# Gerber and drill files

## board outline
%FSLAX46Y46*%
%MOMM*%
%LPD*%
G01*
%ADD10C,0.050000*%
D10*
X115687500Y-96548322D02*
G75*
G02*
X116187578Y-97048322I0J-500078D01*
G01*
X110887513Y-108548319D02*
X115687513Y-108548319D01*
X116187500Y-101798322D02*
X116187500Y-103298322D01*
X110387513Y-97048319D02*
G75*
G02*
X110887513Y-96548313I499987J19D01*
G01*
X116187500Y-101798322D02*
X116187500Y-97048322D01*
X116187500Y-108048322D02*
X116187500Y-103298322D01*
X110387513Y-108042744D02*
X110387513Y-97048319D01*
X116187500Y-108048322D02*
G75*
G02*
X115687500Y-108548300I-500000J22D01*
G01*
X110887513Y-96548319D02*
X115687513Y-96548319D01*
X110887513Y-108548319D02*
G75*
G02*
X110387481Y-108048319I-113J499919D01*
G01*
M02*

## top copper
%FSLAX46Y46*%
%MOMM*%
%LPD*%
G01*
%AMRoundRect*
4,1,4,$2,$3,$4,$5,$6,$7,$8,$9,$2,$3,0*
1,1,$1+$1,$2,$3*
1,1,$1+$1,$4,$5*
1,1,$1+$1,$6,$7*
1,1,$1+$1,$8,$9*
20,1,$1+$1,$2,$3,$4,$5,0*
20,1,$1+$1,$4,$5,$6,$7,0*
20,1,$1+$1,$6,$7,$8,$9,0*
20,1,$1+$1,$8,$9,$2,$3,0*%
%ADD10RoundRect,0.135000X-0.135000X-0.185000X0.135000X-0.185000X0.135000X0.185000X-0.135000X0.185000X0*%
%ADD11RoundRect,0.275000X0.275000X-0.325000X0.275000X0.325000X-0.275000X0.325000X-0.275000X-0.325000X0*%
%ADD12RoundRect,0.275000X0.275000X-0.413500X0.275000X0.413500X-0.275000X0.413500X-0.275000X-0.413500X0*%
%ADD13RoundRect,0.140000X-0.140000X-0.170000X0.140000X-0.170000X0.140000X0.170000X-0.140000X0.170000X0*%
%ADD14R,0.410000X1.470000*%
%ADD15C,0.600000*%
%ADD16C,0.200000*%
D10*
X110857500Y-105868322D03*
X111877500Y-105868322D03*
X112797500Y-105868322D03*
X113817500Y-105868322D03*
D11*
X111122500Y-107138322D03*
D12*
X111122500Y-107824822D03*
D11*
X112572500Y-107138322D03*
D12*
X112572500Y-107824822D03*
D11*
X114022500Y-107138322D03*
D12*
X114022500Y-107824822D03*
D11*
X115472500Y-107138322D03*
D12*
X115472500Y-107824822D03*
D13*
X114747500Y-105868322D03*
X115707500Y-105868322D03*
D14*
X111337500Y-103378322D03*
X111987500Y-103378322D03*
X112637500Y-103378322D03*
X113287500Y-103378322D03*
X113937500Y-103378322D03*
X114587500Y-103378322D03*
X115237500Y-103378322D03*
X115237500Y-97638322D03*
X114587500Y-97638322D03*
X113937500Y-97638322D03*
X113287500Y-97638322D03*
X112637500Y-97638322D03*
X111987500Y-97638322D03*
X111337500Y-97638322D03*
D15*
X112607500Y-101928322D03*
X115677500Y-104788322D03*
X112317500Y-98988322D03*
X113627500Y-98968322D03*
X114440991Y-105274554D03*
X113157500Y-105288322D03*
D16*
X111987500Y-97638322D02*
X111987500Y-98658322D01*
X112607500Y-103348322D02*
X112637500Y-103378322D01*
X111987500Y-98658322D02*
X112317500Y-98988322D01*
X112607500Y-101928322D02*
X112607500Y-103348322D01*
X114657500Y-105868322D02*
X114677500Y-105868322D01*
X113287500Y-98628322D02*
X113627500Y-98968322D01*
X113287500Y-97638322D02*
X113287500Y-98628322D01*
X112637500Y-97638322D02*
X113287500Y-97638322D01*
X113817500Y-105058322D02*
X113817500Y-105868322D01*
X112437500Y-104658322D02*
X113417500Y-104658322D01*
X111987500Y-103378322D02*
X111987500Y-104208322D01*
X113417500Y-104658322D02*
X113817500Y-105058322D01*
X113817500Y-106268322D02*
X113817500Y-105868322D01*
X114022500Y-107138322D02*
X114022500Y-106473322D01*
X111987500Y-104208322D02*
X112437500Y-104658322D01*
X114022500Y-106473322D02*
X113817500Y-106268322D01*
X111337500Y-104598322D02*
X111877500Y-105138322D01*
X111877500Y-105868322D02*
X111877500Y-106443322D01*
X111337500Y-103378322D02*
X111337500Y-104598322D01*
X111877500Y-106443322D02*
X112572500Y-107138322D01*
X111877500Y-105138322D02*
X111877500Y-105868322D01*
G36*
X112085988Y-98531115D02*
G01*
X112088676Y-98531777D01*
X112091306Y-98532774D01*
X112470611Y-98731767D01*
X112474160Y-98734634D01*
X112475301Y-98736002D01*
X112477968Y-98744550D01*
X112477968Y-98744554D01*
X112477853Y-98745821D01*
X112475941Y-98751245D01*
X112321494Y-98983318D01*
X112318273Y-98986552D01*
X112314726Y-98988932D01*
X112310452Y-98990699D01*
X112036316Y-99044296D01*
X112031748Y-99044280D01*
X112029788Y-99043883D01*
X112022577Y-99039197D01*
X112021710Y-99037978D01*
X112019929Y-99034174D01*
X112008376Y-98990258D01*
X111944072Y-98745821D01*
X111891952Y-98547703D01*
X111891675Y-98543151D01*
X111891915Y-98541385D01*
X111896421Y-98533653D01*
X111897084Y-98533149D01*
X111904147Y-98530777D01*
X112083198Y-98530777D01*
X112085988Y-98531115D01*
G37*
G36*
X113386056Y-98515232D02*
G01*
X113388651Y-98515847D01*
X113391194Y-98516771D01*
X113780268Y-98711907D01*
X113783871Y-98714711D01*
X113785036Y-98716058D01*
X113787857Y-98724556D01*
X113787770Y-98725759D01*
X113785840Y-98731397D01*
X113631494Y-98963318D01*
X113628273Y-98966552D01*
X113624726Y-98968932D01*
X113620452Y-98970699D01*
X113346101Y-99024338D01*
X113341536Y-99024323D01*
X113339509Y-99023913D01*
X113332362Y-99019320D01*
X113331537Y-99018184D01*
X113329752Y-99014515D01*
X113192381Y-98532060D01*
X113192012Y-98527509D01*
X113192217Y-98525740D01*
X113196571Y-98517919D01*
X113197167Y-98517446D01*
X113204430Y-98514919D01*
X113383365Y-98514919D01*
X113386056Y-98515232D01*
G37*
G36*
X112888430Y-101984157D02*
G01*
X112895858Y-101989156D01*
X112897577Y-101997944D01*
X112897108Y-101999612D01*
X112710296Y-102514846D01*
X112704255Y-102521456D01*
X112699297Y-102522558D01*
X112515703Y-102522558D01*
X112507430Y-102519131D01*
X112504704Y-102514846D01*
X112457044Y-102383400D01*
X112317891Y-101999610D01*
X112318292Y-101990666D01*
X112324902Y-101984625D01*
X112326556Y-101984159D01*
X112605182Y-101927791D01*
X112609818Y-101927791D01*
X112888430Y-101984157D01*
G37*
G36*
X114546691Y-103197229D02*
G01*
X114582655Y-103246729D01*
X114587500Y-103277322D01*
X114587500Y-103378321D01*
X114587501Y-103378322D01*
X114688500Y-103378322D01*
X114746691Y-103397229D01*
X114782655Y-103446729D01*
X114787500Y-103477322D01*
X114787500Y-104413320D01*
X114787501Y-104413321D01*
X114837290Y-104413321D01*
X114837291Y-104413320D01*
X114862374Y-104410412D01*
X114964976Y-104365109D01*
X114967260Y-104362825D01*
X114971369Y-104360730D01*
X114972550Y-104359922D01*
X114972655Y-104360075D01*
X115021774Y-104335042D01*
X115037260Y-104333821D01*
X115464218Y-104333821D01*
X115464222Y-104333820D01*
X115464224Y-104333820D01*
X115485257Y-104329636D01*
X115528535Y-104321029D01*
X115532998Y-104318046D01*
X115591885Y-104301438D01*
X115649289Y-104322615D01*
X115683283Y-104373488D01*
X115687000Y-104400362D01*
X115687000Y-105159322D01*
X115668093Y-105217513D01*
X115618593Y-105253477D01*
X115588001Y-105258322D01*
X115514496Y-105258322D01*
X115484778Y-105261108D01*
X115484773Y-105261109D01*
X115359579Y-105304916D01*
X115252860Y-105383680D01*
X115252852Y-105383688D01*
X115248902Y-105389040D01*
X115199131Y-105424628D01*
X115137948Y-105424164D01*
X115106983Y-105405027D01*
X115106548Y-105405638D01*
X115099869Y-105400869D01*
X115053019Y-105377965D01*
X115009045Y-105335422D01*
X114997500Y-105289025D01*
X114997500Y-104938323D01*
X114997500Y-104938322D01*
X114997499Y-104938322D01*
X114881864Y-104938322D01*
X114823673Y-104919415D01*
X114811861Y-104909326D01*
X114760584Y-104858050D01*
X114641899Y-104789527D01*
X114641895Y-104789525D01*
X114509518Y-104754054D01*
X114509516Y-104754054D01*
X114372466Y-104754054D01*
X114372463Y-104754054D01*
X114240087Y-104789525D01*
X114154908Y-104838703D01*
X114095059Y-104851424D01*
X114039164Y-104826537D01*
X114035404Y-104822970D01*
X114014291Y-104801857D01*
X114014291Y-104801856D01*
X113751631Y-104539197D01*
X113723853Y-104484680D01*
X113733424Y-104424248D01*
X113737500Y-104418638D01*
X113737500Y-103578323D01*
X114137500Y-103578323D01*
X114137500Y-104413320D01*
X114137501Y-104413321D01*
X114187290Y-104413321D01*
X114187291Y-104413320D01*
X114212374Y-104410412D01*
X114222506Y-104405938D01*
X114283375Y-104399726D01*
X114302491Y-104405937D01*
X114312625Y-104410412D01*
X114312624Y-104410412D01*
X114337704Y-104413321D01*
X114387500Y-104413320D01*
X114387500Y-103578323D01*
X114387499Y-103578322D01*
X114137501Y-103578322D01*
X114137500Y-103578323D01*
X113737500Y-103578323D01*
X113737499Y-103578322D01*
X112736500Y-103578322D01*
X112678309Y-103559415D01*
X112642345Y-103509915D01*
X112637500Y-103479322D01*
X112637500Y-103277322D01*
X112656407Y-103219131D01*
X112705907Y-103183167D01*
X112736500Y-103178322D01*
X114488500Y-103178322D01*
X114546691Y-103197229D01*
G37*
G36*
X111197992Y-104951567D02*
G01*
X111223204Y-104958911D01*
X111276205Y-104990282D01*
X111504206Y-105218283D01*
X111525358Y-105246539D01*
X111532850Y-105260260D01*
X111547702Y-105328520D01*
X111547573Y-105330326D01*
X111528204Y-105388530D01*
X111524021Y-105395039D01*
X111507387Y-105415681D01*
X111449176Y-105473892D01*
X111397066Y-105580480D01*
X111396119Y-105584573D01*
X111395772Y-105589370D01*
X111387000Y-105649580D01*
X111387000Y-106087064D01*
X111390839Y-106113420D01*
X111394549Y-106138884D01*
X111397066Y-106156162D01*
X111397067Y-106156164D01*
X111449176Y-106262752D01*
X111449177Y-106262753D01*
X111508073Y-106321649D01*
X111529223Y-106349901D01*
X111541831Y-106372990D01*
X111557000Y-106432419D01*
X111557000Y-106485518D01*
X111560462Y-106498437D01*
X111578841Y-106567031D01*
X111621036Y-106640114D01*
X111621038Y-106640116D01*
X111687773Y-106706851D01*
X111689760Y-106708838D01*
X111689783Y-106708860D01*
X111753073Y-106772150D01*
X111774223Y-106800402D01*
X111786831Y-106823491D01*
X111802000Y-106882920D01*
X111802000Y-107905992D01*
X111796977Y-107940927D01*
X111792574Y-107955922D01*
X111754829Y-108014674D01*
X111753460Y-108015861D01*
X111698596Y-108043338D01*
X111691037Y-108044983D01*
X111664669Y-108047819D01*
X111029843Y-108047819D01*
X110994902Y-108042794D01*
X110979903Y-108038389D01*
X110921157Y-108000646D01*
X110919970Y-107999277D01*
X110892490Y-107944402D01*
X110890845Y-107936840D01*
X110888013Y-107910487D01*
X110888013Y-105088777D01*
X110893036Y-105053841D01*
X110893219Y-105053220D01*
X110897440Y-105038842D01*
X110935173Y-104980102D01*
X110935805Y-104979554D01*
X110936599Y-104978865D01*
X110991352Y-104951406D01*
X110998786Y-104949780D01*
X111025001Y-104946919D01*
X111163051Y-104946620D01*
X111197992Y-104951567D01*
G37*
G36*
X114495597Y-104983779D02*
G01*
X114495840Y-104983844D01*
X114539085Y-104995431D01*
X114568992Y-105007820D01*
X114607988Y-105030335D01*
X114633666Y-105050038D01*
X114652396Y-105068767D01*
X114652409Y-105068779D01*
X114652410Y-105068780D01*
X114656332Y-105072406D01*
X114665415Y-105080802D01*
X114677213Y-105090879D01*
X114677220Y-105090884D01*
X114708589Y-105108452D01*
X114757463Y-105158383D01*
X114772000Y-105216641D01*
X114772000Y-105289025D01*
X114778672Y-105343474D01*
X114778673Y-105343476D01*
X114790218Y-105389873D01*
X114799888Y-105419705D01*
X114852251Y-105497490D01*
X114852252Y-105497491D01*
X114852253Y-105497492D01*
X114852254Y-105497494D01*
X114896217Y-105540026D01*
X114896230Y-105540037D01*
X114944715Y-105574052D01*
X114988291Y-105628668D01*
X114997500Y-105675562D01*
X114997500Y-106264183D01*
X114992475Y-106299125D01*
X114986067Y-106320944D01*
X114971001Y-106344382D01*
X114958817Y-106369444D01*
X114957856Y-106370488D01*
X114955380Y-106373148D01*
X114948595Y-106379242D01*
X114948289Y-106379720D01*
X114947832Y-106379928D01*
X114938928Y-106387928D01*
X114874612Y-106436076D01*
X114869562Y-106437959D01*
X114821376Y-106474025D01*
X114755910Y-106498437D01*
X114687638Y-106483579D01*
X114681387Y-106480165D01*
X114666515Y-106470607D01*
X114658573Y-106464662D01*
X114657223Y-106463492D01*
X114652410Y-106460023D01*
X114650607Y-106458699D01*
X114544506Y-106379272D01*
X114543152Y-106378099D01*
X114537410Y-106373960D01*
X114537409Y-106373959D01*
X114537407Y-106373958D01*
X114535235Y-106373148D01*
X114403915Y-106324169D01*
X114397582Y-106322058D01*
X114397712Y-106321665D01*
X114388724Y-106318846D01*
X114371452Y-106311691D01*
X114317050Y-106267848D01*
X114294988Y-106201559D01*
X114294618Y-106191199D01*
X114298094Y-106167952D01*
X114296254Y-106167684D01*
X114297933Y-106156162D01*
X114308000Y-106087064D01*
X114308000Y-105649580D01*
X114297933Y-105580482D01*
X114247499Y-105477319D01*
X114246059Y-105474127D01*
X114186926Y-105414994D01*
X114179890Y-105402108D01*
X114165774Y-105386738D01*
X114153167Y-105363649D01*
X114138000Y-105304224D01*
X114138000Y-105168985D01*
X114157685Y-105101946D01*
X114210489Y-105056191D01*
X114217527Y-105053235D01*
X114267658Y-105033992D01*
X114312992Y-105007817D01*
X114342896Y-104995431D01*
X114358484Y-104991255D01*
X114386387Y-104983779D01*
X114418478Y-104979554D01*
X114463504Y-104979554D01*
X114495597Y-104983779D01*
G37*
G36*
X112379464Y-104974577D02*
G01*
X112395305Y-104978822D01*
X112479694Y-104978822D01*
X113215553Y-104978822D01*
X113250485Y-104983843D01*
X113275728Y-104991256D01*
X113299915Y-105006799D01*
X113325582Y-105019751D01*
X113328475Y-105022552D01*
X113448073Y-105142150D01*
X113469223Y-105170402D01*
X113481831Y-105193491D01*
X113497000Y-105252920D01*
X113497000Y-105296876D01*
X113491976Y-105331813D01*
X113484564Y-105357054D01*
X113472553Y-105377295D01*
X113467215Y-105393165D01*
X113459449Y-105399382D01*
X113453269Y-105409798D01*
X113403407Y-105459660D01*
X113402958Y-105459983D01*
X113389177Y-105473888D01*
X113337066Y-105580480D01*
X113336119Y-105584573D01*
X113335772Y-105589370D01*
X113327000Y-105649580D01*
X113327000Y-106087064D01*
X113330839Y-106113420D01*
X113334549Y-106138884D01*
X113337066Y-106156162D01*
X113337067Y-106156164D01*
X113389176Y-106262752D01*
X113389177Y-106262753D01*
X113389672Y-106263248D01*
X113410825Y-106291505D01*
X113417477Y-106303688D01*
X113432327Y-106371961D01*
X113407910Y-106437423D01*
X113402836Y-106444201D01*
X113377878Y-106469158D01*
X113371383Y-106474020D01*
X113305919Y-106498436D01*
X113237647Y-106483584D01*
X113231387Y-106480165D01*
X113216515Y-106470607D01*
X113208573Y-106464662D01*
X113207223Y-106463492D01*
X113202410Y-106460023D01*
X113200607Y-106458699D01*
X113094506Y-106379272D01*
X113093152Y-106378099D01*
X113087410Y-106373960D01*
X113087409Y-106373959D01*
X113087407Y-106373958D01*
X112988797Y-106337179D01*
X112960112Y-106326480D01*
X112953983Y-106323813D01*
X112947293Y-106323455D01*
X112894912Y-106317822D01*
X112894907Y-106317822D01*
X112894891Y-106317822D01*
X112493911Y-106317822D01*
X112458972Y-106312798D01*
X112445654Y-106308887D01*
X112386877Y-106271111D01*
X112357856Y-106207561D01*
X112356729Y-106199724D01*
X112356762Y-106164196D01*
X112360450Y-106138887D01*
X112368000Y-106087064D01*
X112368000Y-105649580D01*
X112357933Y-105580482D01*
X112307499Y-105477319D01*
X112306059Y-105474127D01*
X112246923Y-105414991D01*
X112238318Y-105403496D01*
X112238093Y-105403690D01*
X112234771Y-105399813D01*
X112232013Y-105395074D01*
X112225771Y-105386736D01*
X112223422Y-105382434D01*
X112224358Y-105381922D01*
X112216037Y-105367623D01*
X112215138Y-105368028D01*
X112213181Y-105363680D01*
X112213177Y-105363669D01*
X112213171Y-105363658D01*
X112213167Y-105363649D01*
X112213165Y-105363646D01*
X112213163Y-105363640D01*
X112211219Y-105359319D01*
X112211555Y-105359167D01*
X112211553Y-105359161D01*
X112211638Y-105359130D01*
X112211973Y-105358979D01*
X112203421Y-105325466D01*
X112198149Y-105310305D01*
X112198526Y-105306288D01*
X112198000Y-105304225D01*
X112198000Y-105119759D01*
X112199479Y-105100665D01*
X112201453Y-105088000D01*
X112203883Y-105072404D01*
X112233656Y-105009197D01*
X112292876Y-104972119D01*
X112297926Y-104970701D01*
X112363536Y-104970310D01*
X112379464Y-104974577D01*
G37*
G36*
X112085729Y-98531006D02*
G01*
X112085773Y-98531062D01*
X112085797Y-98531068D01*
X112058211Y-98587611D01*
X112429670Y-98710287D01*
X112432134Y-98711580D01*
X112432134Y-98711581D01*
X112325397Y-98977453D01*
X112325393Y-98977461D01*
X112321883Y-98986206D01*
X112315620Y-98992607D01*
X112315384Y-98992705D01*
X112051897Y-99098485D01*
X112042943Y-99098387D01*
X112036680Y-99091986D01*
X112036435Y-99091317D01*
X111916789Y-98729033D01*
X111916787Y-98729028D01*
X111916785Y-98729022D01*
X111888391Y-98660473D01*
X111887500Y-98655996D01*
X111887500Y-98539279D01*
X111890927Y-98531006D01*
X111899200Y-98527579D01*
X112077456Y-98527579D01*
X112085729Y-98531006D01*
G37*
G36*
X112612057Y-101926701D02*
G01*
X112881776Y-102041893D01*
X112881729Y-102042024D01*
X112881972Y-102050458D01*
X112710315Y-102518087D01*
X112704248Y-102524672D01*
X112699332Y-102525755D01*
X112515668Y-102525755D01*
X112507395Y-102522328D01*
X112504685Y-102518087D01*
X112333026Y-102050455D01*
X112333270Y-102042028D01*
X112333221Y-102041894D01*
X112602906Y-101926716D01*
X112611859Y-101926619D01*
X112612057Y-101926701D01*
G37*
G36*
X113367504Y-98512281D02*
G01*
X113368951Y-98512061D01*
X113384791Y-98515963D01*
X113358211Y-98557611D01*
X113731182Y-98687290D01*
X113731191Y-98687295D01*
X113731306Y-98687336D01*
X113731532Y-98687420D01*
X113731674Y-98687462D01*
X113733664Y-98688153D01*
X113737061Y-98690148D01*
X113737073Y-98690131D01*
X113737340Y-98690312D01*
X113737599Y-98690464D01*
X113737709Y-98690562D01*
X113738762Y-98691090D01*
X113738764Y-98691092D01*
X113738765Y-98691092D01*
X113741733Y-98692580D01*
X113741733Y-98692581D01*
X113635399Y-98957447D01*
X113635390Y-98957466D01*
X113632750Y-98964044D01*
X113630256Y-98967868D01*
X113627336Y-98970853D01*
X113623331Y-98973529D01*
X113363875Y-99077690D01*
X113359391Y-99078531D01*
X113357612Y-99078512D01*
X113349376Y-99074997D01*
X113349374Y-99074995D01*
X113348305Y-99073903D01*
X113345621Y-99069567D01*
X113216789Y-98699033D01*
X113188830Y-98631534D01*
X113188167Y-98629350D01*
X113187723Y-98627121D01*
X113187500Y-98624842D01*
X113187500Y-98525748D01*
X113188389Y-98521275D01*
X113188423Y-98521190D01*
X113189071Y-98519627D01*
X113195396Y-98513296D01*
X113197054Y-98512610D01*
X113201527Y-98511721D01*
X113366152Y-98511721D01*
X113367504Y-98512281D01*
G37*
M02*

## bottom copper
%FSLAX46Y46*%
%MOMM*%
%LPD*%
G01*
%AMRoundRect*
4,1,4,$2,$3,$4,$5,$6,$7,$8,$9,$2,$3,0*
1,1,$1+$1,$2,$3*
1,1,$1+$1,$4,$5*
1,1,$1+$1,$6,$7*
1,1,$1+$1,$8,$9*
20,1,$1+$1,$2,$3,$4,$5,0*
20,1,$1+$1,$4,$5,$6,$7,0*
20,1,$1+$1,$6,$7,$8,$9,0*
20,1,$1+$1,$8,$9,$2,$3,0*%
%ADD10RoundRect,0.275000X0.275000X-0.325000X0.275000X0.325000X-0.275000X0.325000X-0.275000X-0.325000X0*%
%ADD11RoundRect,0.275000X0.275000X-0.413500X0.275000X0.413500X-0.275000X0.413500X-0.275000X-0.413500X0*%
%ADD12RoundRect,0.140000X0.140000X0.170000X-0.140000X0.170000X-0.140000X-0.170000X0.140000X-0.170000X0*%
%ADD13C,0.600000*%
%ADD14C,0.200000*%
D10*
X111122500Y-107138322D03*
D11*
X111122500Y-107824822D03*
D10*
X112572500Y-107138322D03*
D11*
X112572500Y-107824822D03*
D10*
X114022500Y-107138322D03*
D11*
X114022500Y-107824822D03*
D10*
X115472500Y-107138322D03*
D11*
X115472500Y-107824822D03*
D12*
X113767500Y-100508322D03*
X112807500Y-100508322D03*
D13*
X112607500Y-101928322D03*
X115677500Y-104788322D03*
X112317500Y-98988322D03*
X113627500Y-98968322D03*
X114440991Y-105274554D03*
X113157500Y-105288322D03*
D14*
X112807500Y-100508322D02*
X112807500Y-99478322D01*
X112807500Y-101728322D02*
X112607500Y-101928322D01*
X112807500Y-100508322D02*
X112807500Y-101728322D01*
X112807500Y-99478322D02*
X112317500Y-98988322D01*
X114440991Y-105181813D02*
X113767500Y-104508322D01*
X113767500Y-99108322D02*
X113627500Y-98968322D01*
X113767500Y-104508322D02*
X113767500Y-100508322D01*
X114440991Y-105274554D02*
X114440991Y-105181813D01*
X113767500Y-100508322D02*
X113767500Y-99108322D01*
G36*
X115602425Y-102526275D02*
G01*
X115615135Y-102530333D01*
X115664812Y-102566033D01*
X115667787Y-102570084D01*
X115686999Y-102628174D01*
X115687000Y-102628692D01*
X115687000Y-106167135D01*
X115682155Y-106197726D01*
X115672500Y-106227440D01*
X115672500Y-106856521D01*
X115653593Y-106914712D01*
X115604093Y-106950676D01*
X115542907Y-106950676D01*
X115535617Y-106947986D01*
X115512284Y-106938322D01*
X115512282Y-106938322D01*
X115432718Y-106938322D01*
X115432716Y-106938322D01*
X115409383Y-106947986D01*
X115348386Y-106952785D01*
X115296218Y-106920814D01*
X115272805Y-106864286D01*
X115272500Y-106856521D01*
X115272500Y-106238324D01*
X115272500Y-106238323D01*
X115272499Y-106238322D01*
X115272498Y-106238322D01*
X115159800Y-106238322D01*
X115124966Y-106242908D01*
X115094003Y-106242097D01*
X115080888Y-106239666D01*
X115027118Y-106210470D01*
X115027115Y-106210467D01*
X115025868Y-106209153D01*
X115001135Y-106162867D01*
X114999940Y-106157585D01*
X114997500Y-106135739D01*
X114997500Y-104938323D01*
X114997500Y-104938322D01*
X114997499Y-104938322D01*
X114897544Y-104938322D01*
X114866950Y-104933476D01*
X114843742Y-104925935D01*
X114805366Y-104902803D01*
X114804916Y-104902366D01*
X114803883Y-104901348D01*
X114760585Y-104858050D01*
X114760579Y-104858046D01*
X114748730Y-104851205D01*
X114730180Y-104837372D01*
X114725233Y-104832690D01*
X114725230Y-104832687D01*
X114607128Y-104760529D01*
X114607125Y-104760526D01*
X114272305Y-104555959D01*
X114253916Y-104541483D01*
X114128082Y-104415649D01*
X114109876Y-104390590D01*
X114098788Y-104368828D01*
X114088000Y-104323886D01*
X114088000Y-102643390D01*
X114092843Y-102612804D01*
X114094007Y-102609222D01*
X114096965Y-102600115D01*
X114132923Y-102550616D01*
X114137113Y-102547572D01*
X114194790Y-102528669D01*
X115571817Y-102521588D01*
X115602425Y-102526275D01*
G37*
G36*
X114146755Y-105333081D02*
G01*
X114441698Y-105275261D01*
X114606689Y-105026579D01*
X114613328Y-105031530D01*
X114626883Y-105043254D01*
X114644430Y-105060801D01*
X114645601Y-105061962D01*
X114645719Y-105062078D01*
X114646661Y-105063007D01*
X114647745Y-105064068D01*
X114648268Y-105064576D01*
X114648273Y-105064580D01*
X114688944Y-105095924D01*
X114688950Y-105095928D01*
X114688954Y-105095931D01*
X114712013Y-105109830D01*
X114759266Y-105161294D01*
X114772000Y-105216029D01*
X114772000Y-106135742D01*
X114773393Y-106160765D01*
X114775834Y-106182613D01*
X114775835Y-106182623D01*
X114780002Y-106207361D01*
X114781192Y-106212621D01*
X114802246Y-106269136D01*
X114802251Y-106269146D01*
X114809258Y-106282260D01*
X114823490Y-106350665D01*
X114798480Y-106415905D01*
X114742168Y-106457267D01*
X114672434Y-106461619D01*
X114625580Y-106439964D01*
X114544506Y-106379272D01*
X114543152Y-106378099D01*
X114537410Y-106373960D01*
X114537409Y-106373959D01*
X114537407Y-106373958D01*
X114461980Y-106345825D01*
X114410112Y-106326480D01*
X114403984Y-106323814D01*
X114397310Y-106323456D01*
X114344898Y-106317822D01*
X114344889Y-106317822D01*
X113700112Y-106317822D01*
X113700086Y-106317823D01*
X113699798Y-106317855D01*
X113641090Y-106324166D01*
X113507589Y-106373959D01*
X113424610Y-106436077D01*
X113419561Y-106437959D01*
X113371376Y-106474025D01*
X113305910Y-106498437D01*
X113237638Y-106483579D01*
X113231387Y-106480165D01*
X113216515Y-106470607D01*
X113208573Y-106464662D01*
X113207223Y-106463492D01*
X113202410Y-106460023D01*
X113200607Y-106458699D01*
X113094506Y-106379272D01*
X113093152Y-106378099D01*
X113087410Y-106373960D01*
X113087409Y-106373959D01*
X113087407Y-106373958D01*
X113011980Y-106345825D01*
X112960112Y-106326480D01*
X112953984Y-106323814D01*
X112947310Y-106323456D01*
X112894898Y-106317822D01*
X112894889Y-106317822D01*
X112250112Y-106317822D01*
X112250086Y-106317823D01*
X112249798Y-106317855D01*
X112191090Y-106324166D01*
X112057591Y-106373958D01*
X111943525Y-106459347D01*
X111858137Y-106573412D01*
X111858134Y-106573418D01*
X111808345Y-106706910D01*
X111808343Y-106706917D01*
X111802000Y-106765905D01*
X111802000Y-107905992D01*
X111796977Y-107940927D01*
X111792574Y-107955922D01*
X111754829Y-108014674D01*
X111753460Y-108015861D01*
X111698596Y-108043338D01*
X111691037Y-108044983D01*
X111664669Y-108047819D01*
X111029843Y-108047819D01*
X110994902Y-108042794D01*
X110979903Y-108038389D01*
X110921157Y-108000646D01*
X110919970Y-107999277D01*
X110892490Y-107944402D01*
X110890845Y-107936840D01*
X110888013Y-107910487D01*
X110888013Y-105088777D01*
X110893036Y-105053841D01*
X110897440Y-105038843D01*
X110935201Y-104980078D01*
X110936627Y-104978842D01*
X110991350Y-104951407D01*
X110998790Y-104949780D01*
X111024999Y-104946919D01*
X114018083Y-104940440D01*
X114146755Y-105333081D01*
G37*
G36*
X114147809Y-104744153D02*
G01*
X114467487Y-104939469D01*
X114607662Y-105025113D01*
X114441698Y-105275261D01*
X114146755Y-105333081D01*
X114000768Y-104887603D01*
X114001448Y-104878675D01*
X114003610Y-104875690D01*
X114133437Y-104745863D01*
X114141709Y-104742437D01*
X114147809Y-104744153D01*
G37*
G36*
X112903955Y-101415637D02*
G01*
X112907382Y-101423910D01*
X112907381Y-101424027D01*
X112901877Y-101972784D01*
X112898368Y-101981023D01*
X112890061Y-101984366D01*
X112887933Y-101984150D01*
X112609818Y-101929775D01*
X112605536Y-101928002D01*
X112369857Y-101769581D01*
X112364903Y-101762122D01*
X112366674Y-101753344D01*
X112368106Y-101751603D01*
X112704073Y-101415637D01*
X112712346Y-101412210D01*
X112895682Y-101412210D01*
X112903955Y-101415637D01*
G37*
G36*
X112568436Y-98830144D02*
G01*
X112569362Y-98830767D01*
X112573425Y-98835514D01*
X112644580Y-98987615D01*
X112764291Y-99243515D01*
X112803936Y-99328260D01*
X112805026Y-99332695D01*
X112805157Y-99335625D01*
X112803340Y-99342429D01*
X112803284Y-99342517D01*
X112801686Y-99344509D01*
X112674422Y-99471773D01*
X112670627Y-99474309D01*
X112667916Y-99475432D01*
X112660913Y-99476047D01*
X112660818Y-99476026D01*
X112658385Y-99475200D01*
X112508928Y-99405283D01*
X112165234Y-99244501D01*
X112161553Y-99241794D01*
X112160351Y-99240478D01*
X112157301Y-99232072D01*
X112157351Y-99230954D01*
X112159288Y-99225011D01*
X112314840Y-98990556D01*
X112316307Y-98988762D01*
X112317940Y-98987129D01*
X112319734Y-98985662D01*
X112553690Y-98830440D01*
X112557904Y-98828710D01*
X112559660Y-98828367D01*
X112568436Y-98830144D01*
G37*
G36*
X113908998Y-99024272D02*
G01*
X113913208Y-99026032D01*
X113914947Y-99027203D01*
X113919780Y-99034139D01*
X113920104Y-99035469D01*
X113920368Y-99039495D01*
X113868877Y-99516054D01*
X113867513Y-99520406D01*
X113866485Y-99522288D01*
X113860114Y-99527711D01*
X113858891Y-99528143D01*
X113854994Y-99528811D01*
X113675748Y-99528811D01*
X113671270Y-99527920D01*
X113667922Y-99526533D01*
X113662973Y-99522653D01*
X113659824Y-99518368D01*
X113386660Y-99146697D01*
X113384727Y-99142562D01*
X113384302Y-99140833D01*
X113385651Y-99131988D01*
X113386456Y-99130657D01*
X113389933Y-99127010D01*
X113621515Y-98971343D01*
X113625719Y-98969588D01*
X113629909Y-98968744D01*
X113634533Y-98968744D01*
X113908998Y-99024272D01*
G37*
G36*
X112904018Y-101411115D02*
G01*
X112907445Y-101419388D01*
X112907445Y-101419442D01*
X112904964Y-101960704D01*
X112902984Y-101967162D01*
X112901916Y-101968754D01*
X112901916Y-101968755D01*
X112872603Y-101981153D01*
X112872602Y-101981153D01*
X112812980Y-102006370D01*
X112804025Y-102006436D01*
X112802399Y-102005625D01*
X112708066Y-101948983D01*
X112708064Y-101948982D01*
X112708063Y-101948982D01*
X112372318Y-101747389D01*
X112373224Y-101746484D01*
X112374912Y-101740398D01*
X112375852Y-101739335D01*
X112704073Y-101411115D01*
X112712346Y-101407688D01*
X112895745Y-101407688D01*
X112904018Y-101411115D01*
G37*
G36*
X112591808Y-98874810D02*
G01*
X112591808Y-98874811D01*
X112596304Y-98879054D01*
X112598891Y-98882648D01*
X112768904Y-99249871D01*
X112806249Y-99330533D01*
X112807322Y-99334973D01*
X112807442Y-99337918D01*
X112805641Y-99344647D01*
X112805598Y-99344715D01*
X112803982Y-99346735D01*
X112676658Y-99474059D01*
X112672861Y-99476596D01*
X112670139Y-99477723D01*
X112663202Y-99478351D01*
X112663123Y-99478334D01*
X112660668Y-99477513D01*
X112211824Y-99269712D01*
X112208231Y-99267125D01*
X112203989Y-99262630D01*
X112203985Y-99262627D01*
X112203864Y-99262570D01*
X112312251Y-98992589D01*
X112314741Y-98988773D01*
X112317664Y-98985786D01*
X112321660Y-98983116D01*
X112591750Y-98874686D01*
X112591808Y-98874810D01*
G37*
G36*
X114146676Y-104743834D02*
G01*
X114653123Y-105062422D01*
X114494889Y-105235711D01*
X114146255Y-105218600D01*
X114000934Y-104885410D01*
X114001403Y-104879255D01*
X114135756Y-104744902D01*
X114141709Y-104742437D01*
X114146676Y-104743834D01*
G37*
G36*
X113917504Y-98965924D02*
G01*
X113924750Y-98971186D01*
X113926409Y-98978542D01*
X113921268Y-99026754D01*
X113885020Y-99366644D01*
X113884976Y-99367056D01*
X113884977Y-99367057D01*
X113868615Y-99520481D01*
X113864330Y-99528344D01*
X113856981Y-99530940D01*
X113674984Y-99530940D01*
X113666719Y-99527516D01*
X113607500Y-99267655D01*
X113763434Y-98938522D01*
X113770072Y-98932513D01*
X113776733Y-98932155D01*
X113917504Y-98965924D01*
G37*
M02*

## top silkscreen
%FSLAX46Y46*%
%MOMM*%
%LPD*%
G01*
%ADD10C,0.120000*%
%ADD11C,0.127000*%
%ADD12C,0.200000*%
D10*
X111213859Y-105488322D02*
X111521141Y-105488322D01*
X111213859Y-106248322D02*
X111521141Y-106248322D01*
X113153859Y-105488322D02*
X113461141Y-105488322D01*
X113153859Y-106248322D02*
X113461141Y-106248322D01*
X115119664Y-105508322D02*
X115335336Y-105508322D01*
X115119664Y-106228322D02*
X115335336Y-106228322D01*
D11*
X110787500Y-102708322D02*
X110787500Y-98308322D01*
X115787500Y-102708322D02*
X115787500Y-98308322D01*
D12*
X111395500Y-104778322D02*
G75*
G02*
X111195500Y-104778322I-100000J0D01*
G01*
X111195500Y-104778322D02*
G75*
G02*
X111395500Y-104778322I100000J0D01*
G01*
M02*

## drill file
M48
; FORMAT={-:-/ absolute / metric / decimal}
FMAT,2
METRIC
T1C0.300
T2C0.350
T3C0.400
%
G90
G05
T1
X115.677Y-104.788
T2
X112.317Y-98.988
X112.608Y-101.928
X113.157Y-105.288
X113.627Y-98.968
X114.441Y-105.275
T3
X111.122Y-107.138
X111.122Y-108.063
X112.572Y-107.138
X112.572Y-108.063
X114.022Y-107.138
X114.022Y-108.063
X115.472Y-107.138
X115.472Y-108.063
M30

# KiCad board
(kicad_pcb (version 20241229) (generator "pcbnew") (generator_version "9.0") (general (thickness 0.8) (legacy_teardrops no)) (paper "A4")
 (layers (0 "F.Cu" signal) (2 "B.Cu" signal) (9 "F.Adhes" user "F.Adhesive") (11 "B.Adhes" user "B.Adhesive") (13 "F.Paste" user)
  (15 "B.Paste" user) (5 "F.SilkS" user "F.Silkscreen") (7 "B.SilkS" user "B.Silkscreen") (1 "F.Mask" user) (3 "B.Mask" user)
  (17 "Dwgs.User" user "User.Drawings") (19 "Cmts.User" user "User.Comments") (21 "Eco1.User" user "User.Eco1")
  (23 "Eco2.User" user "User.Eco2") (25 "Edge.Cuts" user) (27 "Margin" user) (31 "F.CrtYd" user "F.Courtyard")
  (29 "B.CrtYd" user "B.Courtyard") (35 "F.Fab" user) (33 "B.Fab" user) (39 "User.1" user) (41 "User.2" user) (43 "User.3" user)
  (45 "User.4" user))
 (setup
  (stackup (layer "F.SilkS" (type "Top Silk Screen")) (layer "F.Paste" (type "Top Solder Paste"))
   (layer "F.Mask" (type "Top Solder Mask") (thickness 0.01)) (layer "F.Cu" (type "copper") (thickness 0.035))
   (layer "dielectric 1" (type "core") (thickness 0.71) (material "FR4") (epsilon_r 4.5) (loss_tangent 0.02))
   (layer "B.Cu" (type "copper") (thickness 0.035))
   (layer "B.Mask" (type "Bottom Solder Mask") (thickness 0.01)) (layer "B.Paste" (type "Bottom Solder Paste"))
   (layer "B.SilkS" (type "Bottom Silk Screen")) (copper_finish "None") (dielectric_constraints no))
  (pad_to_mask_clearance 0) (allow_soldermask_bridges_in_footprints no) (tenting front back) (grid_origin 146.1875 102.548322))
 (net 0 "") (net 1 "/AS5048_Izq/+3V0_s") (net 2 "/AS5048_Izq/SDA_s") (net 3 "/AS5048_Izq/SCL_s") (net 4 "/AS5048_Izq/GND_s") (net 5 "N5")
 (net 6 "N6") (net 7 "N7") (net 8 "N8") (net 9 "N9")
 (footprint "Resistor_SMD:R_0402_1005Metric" (layer "F.Cu") (at 111.3675 105.868322)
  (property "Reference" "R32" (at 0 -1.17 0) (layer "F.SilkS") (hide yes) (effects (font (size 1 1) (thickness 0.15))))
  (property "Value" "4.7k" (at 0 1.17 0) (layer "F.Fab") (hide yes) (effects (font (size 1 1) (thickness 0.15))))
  (fp_line (start -0.153641 -0.38) (end 0.153641 -0.38) (stroke (width 0.12) (type solid)) (layer "F.SilkS"))
  (fp_line (start -0.153641 0.38) (end 0.153641 0.38) (stroke (width 0.12) (type solid)) (layer "F.SilkS"))
  (pad "1" smd roundrect (at -0.51 0) (size 0.54 0.64) (layers "F.Cu" "F.Mask" "F.Paste") (roundrect_rratio 0.25)
   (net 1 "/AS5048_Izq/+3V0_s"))
  (pad "2" smd roundrect (at 0.51 0) (size 0.54 0.64) (layers "F.Cu" "F.Mask" "F.Paste") (roundrect_rratio 0.25) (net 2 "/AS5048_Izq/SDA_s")))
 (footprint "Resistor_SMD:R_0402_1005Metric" (layer "F.Cu") (at 113.3075 105.868322)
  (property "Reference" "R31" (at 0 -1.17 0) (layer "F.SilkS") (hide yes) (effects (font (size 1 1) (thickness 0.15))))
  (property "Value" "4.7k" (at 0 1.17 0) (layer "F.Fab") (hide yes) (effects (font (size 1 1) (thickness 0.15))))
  (fp_line (start -0.153641 -0.38) (end 0.153641 -0.38) (stroke (width 0.12) (type solid)) (layer "F.SilkS"))
  (fp_line (start -0.153641 0.38) (end 0.153641 0.38) (stroke (width 0.12) (type solid)) (layer "F.SilkS"))
  (pad "1" smd roundrect (at -0.51 0) (size 0.54 0.64) (layers "F.Cu" "F.Mask" "F.Paste") (roundrect_rratio 0.25)
   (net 1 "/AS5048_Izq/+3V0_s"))
  (pad "2" smd roundrect (at 0.51 0) (size 0.54 0.64) (layers "F.Cu" "F.Mask" "F.Paste") (roundrect_rratio 0.25) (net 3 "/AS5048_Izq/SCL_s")))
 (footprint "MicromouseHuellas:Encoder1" (layer "F.Cu") (at 113.2975 107.138322)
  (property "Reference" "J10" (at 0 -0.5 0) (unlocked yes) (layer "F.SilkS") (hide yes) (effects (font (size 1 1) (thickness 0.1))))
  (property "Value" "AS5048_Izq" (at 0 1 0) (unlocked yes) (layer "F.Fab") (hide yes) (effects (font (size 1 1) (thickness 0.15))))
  (pad "1" thru_hole roundrect (at -2.175 0 90) (size 1.2 1.1) (drill 0.4) (layers "*.Cu" "*.Mask") (remove_unused_layers no)
   (roundrect_rratio 0.25) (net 1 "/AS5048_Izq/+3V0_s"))
  (pad "1" thru_hole roundrect (at -2.175 0.925 90) (size 1.377 1.1) (drill 0.4 (offset 0.2385 0)) (layers "*.Cu" "*.Mask")
   (remove_unused_layers no) (roundrect_rratio 0.25) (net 1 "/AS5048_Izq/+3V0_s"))
  (pad "2" thru_hole roundrect (at -0.725 0 90) (size 1.2 1.1) (drill 0.4) (layers "*.Cu" "*.Mask") (remove_unused_layers no)
   (roundrect_rratio 0.25) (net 2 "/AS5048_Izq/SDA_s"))
  (pad "2" thru_hole roundrect (at -0.725 0.925 90) (size 1.377 1.1) (drill 0.4 (offset 0.2385 0)) (layers "*.Cu" "*.Mask")
   (remove_unused_layers no) (roundrect_rratio 0.25) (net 2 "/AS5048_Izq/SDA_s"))
  (pad "3" thru_hole roundrect (at 0.725 0 90) (size 1.2 1.1) (drill 0.4) (layers "*.Cu" "*.Mask") (remove_unused_layers no)
   (roundrect_rratio 0.25) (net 3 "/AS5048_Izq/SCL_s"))
  (pad "3" thru_hole roundrect (at 0.725 0.925 90) (size 1.377 1.1) (drill 0.4 (offset 0.2385 0)) (layers "*.Cu" "*.Mask")
   (remove_unused_layers no) (roundrect_rratio 0.25) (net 3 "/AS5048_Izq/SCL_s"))
  (pad "4" thru_hole roundrect (at 2.175 0 90) (size 1.2 1.1) (drill 0.4) (layers "*.Cu" "*.Mask") (remove_unused_layers no)
   (roundrect_rratio 0.25) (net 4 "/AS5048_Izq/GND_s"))
  (pad "4" thru_hole roundrect (at 2.175 0.925 90) (size 1.377 1.1) (drill 0.4 (offset 0.2385 0)) (layers "*.Cu" "*.Mask")
   (remove_unused_layers no) (roundrect_rratio 0.25) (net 4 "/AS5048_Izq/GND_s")))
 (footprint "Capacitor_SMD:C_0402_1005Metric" (layer "F.Cu") (at 115.2275 105.868322)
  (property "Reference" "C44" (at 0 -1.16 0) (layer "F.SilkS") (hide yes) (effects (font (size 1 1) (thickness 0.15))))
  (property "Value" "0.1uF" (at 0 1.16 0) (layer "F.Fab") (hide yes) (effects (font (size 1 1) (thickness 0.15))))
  (fp_line (start -0.107836 -0.36) (end 0.107836 -0.36) (stroke (width 0.12) (type solid)) (layer "F.SilkS"))
  (fp_line (start -0.107836 0.36) (end 0.107836 0.36) (stroke (width 0.12) (type solid)) (layer "F.SilkS"))
  (pad "1" smd roundrect (at -0.48 0) (size 0.56 0.62) (layers "F.Cu" "F.Mask" "F.Paste") (roundrect_rratio 0.25)
   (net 1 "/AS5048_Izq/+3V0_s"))
  (pad "2" smd roundrect (at 0.48 0) (size 0.56 0.62) (layers "F.Cu" "F.Mask" "F.Paste") (roundrect_rratio 0.25) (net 4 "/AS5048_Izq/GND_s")))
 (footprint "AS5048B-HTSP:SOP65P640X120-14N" (layer "F.Cu") (at 113.2875 100.508322 90)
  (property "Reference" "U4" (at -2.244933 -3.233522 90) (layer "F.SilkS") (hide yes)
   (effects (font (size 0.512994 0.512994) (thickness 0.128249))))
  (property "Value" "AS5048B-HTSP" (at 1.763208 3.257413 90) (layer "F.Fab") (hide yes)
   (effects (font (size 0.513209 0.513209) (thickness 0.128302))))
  (fp_line (start -2.2 -2.5) (end 2.2 -2.5) (stroke (width 0.127) (type solid)) (layer "F.SilkS"))
  (fp_line (start -2.2 2.5) (end 2.2 2.5) (stroke (width 0.127) (type solid)) (layer "F.SilkS"))
  (fp_circle (center -4.27 -1.992) (end -4.17 -1.992) (stroke (width 0.2) (type solid)) (fill no) (layer "F.SilkS"))
  (pad "1" smd rect (at -2.87 -1.95 90) (size 1.47 0.41) (layers "F.Cu" "F.Mask" "F.Paste") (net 2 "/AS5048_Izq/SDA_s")
   (solder_mask_margin 0.102))
  (pad "2" smd rect (at -2.87 -1.3 90) (size 1.47 0.41) (layers "F.Cu" "F.Mask" "F.Paste") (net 3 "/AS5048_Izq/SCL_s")
   (solder_mask_margin 0.102))
  (pad "3" smd rect (at -2.87 -0.65 90) (size 1.47 0.41) (layers "F.Cu" "F.Mask" "F.Paste") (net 4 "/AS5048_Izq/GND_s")
   (solder_mask_margin 0.102))
  (pad "4" smd rect (at -2.87 0 90) (size 1.47 0.41) (layers "F.Cu" "F.Mask" "F.Paste") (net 4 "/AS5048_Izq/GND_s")
   (solder_mask_margin 0.102))
  (pad "5" smd rect (at -2.87 0.65 90) (size 1.47 0.41) (layers "F.Cu" "F.Mask" "F.Paste") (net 4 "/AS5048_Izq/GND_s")
   (solder_mask_margin 0.102))
  (pad "6" smd rect (at -2.87 1.3 90) (size 1.47 0.41) (layers "F.Cu" "F.Mask" "F.Paste") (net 4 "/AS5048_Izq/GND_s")
   (solder_mask_margin 0.102))
  (pad "7" smd rect (at -2.87 1.95 90) (size 1.47 0.41) (layers "F.Cu" "F.Mask" "F.Paste") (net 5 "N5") (solder_mask_margin 0.102))
  (pad "8" smd rect (at 2.87 1.95 90) (size 1.47 0.41) (layers "F.Cu" "F.Mask" "F.Paste") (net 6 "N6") (solder_mask_margin 0.102))
  (pad "9" smd rect (at 2.87 1.3 90) (size 1.47 0.41) (layers "F.Cu" "F.Mask" "F.Paste") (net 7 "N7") (solder_mask_margin 0.102))
  (pad "10" smd rect (at 2.87 0.65 90) (size 1.47 0.41) (layers "F.Cu" "F.Mask" "F.Paste") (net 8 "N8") (solder_mask_margin 0.102))
  (pad "11" smd rect (at 2.87 0 90) (size 1.47 0.41) (layers "F.Cu" "F.Mask" "F.Paste") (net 1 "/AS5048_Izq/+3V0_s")
   (solder_mask_margin 0.102))
  (pad "12" smd rect (at 2.87 -0.65 90) (size 1.47 0.41) (layers "F.Cu" "F.Mask" "F.Paste") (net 1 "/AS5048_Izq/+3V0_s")
   (solder_mask_margin 0.102))
  (pad "13" smd rect (at 2.87 -1.3 90) (size 1.47 0.41) (layers "F.Cu" "F.Mask" "F.Paste") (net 4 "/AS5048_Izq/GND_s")
   (solder_mask_margin 0.102))
  (pad "14" smd rect (at 2.87 -1.95 90) (size 1.47 0.41) (layers "F.Cu" "F.Mask" "F.Paste") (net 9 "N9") (solder_mask_margin 0.102)))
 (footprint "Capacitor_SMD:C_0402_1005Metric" (layer "B.Cu") (at 113.2875 100.508322 180)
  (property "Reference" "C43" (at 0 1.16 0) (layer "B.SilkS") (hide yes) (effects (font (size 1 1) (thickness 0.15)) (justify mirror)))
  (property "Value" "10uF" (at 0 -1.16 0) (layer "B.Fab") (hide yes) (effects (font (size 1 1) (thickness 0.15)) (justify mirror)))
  (pad "1" smd roundrect (at -0.48 0 180) (size 0.56 0.62) (layers "B.Cu" "B.Mask" "B.Paste") (roundrect_rratio 0.25)
   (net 1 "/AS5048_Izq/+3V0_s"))
  (pad "2" smd roundrect (at 0.48 0 180) (size 0.56 0.62) (layers "B.Cu" "B.Mask" "B.Paste") (roundrect_rratio 0.25)
   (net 4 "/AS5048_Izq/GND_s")))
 (gr_arc (start 115.6875 96.548322) (mid 116.041031 96.694772) (end 116.1875 97.048322) (stroke (width 0.05) (type default))
  (layer "Edge.Cuts"))
 (gr_line (start 110.887513 108.548319) (end 115.687513 108.548319) (stroke (width 0.05) (type solid)) (layer "Edge.Cuts"))
 (gr_line (start 116.1875 101.798322) (end 116.1875 103.298322) (stroke (width 0.05) (type default)) (layer "Edge.Cuts"))
 (gr_arc (start 110.387513 97.048319) (mid 110.533968 96.69476) (end 110.887513 96.548319) (stroke (width 0.05) (type default))
  (layer "Edge.Cuts"))
 (gr_line (start 116.1875 101.798322) (end 116.1875 97.048322) (stroke (width 0.05) (type solid)) (layer "Edge.Cuts"))
 (gr_line (start 116.1875 108.048322) (end 116.1875 103.298322) (stroke (width 0.05) (type solid)) (layer "Edge.Cuts"))
 (gr_line (start 110.387513 108.042744) (end 110.387513 97.048319) (stroke (width 0.05) (type default)) (layer "Edge.Cuts"))
 (gr_arc (start 116.1875 108.048322) (mid 116.04106 108.401863) (end 115.6875 108.548322) (stroke (width 0.05) (type default))
  (layer "Edge.Cuts"))
 (gr_line (start 110.887513 96.548319) (end 115.687513 96.548319) (stroke (width 0.05) (type solid)) (layer "Edge.Cuts"))
 (gr_arc (start 110.887513 108.548319) (mid 110.53393 108.401881) (end 110.387513 108.048319) (stroke (width 0.05) (type default))
  (layer "Edge.Cuts"))
 (segment (start 111.9875 97.638322) (end 111.9875 98.658322) (width 0.2) (layer "F.Cu") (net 4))
 (segment (start 112.6075 103.348322) (end 112.6375 103.378322) (width 0.2) (layer "F.Cu") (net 4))
 (segment (start 111.9875 98.658322) (end 112.3175 98.988322) (width 0.2) (layer "F.Cu") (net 4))
 (segment (start 112.6075 101.928322) (end 112.6075 103.348322) (width 0.2) (layer "F.Cu") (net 4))
 (via (at 112.6075 101.928322) (size 0.6) (drill 0.35) (layers "F.Cu" "B.Cu")
  (teardrops (best_length_ratio 0.5) (max_length 1) (best_width_ratio 1) (max_width 2) (curved_edges no) (filter_ratio 0.9) (enabled yes)
   (allow_two_segments yes) (prefer_zone_connections yes))
  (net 4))
 (via (at 115.6775 104.788322) (size 0.6) (drill 0.3) (layers "F.Cu" "B.Cu") (free yes) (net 4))
 (via (at 112.3175 98.988322) (size 0.6) (drill 0.35) (layers "F.Cu" "B.Cu")
  (teardrops (best_length_ratio 0.5) (max_length 1) (best_width_ratio 1) (max_width 2) (curved_edges no) (filter_ratio 0.9) (enabled yes)
   (allow_two_segments yes) (prefer_zone_connections yes))
  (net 4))
 (segment (start 112.8075 100.508322) (end 112.8075 99.478322) (width 0.2) (layer "B.Cu") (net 4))
 (segment (start 112.8075 101.728322) (end 112.6075 101.928322) (width 0.2) (layer "B.Cu") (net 4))
 (segment (start 112.8075 100.508322) (end 112.8075 101.728322) (width 0.2) (layer "B.Cu") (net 4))
 (segment (start 112.8075 99.478322) (end 112.3175 98.988322) (width 0.2) (layer "B.Cu") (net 4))
 (segment (start 114.6575 105.868322) (end 114.6775 105.868322) (width 0.2) (layer "F.Cu") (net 1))
 (segment (start 113.2875 98.628322) (end 113.6275 98.968322) (width 0.2) (layer "F.Cu") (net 1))
 (segment (start 113.2875 97.638322) (end 113.2875 98.628322) (width 0.2) (layer "F.Cu") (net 1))
 (segment (start 112.6375 97.638322) (end 113.2875 97.638322) (width 0.2) (layer "F.Cu") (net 1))
 (via (at 113.6275 98.968322) (size 0.6) (drill 0.35) (layers "F.Cu" "B.Cu")
  (teardrops (best_length_ratio 0.5) (max_length 1) (best_width_ratio 1) (max_width 2) (curved_edges no) (filter_ratio 0.9) (enabled yes)
   (allow_two_segments yes) (prefer_zone_connections yes))
  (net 1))
 (via (at 114.440991 105.274554) (size 0.6) (drill 0.35) (layers "F.Cu" "B.Cu")
  (teardrops (best_length_ratio 0.5) (max_length 1) (best_width_ratio 1) (max_width 2) (curved_edges no) (filter_ratio 0.9) (enabled yes)
   (allow_two_segments yes) (prefer_zone_connections yes))
  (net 1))
 (via (at 113.1575 105.288322) (size 0.6) (drill 0.35) (layers "F.Cu" "B.Cu") (free yes)
  (teardrops (best_length_ratio 0.5) (max_length 1) (best_width_ratio 1) (max_width 2) (curved_edges no) (filter_ratio 0.9) (enabled yes)
   (allow_two_segments yes) (prefer_zone_connections yes))
  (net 1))
 (segment (start 114.440991 105.181813) (end 113.7675 104.508322) (width 0.2) (layer "B.Cu") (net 1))
 (segment (start 113.7675 99.108322) (end 113.6275 98.968322) (width 0.2) (layer "B.Cu") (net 1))
 (segment (start 113.7675 104.508322) (end 113.7675 100.508322) (width 0.2) (layer "B.Cu") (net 1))
 (segment (start 114.440991 105.274554) (end 114.440991 105.181813) (width 0.2) (layer "B.Cu") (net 1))
 (segment (start 113.7675 100.508322) (end 113.7675 99.108322) (width 0.2) (layer "B.Cu") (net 1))
 (segment (start 113.8175 105.058322) (end 113.8175 105.868322) (width 0.2) (layer "F.Cu") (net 3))
 (segment (start 112.4375 104.658322) (end 113.4175 104.658322) (width 0.2) (layer "F.Cu") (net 3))
 (segment (start 111.9875 103.378322) (end 111.9875 104.208322) (width 0.2) (layer "F.Cu") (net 3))
 (segment (start 113.4175 104.658322) (end 113.8175 105.058322) (width 0.2) (layer "F.Cu") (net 3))
 (segment (start 113.8175 106.268322) (end 113.8175 105.868322) (width 0.2) (layer "F.Cu") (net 3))
 (segment (start 114.0225 107.138322) (end 114.0225 106.473322) (width 0.2) (layer "F.Cu") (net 3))
 (segment (start 111.9875 104.208322) (end 112.4375 104.658322) (width 0.2) (layer "F.Cu") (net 3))
 (segment (start 114.0225 106.473322) (end 113.8175 106.268322) (width 0.2) (layer "F.Cu") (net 3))
 (segment (start 111.3375 104.598322) (end 111.8775 105.138322) (width 0.2) (layer "F.Cu") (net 2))
 (segment (start 111.8775 105.868322) (end 111.8775 106.443322) (width 0.2) (layer "F.Cu") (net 2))
 (segment (start 111.3375 103.378322) (end 111.3375 104.598322) (width 0.2) (layer "F.Cu") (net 2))
 (segment (start 111.8775 106.443322) (end 112.5725 107.138322) (width 0.2) (layer "F.Cu") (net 2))
 (segment (start 111.8775 105.138322) (end 111.8775 105.868322) (width 0.2) (layer "F.Cu") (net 2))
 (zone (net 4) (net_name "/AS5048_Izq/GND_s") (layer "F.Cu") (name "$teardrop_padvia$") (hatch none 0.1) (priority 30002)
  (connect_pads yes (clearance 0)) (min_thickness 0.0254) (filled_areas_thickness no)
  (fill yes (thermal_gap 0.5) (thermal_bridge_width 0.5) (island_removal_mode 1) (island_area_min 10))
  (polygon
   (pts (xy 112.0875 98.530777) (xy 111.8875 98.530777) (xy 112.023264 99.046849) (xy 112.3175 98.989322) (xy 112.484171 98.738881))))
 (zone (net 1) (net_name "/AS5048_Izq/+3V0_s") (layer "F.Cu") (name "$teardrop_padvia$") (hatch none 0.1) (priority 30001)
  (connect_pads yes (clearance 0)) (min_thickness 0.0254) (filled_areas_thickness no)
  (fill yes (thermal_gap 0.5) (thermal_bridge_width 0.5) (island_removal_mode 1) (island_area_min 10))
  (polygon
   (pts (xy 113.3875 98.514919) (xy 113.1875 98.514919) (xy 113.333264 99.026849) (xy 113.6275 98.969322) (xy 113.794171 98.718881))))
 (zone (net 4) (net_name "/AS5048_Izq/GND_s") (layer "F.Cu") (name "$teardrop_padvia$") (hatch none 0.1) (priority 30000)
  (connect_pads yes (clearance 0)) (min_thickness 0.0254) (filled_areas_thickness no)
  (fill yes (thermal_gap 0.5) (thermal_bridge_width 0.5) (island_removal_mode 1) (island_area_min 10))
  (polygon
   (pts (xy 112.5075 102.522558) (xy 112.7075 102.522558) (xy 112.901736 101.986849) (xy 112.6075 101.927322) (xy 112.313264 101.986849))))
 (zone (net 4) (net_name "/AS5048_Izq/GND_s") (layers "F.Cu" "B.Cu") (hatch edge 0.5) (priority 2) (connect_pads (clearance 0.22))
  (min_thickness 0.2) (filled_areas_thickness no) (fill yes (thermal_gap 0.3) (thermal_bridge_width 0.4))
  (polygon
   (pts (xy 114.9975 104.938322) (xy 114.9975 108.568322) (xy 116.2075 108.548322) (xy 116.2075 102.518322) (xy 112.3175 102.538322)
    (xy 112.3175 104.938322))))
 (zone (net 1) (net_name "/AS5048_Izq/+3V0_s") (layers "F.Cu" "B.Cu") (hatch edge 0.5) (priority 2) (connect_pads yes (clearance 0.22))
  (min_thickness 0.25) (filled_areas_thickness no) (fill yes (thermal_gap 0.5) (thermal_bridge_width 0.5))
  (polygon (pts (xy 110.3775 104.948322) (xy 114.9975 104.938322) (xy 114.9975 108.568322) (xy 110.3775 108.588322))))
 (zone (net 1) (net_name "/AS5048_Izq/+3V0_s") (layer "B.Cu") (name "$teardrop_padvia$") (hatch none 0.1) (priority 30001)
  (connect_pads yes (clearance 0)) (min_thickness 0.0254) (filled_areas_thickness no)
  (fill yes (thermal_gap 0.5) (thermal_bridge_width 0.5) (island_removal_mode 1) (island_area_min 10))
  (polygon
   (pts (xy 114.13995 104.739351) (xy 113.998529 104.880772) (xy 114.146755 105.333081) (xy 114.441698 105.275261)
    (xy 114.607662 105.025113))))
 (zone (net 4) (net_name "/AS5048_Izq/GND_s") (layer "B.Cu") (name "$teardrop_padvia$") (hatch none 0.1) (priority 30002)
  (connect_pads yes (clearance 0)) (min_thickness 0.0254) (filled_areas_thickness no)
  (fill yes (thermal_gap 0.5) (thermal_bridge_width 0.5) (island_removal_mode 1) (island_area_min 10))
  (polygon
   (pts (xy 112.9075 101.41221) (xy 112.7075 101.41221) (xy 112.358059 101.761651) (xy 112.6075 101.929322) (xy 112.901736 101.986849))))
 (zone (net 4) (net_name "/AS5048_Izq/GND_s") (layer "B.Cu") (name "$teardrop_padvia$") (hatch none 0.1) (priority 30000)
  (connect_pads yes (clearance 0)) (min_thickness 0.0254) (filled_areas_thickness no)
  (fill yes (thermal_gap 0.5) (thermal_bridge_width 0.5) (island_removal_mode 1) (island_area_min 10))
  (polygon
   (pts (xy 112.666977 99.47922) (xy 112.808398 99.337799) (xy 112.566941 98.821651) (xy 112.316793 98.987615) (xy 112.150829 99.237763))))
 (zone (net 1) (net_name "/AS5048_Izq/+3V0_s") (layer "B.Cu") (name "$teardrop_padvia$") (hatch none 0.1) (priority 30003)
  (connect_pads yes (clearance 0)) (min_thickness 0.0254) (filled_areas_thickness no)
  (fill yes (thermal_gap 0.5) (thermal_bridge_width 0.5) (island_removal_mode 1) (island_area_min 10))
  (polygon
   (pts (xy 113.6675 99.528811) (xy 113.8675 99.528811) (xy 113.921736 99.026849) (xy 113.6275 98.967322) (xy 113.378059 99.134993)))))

